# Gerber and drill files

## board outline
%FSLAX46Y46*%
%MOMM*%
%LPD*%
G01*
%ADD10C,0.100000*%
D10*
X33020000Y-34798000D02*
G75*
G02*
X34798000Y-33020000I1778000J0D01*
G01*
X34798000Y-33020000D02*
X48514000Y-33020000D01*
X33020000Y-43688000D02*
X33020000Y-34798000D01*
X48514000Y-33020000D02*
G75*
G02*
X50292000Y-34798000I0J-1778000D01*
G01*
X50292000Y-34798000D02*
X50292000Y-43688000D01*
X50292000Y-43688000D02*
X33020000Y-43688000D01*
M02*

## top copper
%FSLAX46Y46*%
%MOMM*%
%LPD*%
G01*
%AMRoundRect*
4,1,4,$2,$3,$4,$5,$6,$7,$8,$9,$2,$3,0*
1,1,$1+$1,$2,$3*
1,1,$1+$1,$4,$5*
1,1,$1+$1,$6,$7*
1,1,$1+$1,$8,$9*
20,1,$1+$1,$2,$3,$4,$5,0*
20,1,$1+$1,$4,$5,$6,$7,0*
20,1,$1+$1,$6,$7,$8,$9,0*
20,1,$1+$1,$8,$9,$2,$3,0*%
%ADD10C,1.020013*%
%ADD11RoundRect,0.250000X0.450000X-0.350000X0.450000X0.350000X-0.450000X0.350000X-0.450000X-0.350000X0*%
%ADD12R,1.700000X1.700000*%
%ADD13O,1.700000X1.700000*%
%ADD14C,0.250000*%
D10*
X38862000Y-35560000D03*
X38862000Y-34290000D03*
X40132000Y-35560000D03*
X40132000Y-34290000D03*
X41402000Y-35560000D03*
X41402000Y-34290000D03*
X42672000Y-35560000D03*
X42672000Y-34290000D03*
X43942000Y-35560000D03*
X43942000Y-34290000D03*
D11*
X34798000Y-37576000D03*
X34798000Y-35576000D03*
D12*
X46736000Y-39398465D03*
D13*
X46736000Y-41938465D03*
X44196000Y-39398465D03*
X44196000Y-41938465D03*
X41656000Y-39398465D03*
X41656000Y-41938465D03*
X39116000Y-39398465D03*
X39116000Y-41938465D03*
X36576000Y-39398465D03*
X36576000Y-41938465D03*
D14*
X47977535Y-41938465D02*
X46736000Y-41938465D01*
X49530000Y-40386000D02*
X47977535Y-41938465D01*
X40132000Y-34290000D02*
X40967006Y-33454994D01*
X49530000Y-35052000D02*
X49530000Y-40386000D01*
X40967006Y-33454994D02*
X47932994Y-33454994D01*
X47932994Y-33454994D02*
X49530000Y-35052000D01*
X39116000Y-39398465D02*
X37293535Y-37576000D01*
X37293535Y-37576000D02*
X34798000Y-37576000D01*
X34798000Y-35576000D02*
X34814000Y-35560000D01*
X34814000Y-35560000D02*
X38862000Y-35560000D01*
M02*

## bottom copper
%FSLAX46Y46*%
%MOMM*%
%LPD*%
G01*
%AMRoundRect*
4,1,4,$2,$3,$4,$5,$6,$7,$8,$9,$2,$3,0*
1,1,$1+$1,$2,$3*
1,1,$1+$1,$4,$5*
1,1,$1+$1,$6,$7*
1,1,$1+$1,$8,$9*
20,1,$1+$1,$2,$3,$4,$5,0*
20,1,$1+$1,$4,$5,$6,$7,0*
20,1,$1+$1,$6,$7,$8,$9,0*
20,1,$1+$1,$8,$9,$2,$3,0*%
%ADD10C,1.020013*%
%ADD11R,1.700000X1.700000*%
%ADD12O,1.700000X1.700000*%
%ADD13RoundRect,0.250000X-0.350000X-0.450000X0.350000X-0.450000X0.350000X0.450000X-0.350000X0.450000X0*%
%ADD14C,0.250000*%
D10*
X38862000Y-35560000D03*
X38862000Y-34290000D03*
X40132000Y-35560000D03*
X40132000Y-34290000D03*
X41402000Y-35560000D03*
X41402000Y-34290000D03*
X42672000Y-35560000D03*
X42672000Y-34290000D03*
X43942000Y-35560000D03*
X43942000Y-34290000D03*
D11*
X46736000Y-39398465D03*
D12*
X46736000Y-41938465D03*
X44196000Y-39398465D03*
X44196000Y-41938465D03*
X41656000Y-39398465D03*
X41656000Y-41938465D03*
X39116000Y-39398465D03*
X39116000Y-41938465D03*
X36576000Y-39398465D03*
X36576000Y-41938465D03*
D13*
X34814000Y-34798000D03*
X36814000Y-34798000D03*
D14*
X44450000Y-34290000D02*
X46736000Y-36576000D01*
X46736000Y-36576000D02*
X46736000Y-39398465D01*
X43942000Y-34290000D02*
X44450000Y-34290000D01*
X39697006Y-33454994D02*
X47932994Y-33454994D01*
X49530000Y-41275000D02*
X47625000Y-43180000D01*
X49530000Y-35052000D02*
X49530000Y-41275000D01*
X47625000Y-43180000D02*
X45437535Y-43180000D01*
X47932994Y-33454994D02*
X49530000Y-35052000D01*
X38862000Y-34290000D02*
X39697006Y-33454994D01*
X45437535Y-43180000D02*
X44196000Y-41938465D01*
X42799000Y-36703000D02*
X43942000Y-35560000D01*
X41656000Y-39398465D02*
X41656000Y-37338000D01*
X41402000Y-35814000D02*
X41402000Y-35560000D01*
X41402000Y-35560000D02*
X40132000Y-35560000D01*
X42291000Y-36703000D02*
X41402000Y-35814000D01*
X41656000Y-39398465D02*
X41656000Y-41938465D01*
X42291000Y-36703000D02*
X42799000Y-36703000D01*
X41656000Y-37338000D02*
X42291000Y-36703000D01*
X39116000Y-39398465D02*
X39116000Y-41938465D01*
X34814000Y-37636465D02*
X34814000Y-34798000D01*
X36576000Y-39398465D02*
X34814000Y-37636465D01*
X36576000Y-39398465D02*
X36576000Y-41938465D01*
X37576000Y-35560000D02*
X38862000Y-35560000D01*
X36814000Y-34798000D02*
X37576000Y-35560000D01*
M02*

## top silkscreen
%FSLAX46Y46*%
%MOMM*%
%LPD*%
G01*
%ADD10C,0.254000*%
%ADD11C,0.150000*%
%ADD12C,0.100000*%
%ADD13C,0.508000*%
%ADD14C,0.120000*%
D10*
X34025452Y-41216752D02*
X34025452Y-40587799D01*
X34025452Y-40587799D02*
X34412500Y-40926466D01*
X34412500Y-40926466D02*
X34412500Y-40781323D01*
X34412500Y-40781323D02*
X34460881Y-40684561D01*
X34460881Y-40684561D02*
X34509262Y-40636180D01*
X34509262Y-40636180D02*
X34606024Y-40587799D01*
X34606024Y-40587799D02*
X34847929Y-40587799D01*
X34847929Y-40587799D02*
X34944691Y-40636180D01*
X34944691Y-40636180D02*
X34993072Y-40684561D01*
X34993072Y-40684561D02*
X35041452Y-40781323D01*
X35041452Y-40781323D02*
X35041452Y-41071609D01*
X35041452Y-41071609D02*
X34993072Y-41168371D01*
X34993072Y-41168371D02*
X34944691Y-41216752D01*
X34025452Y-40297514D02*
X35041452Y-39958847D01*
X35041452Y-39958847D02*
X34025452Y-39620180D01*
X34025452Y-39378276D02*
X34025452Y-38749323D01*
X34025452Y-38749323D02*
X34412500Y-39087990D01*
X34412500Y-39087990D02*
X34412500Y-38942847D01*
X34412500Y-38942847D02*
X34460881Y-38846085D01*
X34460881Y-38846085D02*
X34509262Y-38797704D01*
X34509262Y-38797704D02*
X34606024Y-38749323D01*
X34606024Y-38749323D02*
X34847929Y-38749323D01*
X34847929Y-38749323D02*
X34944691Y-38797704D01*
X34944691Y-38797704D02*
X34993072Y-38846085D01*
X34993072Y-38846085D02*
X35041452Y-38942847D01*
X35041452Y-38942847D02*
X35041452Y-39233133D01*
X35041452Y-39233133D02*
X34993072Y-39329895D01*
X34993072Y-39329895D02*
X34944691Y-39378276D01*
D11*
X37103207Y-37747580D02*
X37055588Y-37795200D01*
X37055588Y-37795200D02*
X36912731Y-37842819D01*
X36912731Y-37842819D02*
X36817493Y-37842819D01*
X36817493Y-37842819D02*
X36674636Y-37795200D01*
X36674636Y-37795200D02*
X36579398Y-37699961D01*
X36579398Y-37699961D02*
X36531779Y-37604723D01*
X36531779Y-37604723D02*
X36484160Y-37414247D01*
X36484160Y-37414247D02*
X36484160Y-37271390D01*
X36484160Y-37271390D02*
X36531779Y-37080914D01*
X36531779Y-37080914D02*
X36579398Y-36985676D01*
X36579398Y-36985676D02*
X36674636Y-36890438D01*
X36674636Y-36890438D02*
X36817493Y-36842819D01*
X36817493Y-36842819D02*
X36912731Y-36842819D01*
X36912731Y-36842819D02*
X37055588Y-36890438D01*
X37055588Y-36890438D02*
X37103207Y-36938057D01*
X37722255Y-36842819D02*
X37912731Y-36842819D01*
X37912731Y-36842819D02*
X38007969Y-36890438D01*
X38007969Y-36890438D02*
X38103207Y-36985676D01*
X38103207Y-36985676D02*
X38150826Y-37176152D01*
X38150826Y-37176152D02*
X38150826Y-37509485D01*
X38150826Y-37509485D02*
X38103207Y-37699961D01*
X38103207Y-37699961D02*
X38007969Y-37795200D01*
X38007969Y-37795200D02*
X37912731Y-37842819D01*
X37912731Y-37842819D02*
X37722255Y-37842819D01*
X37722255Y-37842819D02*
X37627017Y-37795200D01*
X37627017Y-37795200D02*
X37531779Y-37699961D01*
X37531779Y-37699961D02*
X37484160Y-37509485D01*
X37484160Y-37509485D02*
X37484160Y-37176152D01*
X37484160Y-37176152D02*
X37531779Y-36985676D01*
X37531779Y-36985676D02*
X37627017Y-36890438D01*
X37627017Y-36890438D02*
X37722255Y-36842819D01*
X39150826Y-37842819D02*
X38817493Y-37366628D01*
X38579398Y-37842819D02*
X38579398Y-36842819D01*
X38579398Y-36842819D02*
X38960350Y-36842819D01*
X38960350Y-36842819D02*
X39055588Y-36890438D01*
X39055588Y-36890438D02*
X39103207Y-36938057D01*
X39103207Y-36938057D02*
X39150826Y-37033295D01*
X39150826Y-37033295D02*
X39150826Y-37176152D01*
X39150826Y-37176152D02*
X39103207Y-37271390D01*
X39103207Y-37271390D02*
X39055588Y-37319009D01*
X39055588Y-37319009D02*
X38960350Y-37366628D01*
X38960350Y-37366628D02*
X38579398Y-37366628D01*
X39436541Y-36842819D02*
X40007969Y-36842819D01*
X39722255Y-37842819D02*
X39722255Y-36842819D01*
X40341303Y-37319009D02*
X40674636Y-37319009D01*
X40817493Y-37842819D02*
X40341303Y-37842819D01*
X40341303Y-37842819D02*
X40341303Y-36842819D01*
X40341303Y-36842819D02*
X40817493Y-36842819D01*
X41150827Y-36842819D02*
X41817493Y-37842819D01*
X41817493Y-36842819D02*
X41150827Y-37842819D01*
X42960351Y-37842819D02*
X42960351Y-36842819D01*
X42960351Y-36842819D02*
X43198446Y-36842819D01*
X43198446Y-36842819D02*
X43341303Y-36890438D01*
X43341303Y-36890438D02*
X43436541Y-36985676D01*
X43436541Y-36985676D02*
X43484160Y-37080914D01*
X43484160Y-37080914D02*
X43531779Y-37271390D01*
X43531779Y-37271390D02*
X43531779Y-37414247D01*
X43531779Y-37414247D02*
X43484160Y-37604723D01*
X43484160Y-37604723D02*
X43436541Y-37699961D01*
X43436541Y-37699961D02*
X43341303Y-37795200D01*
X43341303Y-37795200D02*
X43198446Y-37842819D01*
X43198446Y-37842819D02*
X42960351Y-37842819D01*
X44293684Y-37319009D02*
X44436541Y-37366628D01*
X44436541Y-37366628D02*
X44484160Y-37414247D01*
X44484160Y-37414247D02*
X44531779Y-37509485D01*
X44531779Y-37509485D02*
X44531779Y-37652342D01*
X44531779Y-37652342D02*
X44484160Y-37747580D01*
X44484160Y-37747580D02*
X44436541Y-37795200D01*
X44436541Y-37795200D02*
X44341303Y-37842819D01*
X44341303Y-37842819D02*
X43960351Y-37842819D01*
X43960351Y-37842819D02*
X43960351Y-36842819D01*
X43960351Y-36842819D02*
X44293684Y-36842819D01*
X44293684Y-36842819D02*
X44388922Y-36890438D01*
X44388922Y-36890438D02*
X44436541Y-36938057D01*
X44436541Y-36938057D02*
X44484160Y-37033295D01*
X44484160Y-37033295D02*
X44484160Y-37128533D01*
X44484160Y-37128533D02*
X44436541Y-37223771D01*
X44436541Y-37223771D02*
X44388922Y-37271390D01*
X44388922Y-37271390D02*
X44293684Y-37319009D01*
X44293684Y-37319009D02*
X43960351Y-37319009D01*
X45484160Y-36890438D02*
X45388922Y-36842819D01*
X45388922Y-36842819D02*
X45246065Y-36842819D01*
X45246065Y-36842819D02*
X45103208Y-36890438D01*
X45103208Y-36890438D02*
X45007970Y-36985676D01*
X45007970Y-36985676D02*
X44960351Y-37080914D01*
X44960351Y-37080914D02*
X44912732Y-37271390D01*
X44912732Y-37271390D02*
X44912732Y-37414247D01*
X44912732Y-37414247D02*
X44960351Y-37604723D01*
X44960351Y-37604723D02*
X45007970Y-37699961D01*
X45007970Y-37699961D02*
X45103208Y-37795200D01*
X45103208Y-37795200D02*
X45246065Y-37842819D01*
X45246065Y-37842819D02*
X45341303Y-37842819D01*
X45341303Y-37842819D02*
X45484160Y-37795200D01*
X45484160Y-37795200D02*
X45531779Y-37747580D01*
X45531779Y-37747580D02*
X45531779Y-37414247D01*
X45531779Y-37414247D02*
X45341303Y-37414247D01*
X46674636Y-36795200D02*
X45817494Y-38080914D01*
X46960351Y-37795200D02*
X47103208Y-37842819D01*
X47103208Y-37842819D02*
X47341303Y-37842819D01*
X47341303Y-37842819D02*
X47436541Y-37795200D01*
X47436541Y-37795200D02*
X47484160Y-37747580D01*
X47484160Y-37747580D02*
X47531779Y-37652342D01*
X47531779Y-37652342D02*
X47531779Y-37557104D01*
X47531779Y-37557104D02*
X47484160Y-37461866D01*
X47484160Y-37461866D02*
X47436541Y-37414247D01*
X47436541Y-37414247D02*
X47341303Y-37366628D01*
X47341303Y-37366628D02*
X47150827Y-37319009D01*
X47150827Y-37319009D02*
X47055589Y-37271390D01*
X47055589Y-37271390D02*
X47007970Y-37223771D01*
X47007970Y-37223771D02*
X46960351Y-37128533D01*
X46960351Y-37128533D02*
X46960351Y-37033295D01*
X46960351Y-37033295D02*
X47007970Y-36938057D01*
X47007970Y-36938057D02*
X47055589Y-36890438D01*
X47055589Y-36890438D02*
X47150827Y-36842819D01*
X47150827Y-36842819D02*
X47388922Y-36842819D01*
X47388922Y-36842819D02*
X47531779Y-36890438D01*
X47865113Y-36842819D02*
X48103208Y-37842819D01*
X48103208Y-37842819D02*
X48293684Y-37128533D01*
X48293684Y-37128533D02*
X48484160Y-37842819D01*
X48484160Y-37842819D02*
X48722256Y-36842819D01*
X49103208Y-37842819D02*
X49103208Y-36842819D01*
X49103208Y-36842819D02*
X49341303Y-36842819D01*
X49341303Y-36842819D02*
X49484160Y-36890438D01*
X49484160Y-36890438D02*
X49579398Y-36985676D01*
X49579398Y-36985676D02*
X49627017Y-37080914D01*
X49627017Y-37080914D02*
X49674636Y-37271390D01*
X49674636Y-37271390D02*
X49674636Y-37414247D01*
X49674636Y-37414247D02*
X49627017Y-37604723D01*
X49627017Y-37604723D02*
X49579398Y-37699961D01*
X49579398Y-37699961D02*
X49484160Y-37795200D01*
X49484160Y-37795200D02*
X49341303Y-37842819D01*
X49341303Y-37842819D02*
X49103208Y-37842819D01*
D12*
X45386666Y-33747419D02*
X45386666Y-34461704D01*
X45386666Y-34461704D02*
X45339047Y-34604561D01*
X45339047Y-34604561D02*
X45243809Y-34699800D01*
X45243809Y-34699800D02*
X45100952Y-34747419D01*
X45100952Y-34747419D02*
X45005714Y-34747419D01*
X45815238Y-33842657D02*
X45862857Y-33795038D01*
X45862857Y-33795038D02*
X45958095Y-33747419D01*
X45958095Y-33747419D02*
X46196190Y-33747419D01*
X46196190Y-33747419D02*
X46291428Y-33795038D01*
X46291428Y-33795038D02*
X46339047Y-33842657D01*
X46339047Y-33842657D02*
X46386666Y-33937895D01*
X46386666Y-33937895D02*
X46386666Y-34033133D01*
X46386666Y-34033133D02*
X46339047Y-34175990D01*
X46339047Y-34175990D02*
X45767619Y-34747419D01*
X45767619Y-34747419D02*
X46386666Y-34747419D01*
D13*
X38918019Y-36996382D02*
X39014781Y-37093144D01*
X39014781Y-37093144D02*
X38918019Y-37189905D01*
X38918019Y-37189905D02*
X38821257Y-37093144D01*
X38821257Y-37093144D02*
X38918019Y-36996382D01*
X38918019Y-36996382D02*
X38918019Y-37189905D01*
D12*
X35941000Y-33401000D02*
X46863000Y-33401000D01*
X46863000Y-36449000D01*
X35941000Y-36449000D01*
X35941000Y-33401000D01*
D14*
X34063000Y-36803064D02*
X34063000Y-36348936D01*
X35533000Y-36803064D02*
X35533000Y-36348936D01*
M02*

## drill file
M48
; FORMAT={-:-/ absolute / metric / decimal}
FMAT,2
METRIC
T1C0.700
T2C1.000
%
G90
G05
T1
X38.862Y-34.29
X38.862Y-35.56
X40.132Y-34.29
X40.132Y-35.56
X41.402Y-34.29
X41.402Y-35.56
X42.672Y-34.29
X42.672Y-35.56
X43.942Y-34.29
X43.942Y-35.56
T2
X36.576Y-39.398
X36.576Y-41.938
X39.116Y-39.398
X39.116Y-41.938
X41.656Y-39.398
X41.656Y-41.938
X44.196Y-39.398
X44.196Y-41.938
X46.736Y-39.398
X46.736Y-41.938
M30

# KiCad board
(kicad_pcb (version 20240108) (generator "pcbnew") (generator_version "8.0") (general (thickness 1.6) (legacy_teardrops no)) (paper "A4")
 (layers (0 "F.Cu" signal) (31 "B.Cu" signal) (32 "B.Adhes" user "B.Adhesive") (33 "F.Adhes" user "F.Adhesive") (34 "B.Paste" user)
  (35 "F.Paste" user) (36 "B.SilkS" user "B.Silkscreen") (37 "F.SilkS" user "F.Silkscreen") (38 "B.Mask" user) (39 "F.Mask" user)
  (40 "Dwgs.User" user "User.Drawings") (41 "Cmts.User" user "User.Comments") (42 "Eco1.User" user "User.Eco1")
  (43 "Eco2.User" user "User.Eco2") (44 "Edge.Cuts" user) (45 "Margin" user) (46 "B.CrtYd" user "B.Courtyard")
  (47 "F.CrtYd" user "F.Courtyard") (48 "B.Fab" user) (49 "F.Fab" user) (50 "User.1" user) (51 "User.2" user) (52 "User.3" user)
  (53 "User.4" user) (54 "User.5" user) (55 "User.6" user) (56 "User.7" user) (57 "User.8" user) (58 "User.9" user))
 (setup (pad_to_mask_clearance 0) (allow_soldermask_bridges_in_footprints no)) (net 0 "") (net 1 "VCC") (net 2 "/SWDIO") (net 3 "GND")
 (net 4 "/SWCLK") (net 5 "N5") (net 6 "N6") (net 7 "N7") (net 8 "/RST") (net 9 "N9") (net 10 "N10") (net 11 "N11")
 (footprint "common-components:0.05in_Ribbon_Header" (layer "F.Cu") (at 41.402 34.925)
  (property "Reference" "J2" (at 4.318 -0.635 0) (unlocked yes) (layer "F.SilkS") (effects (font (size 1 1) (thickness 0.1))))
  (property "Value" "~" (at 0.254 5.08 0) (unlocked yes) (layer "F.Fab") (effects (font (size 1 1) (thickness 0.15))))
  (fp_rect (start -5.461 -1.524) (end 5.461 1.524) (stroke (width 0.1) (type default)) (fill none) (layer "F.SilkS"))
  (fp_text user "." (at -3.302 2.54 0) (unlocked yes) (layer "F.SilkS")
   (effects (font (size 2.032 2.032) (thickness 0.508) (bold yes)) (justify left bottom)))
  (pad "1" thru_hole circle (at -2.54 0.635) (size 1.020013 1.020013) (drill 0.699999) (layers "*.Cu" "*.Mask") (remove_unused_layers no)
   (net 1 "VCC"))
  (pad "2" thru_hole circle (at -2.54 -0.635) (size 1.020013 1.020013) (drill 0.699999) (layers "*.Cu" "*.Mask") (remove_unused_layers no)
   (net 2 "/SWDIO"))
  (pad "3" thru_hole circle (at -1.27 0.635) (size 1.020013 1.020013) (drill 0.699999) (layers "*.Cu" "*.Mask") (remove_unused_layers no)
   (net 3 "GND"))
  (pad "4" thru_hole circle (at -1.27 -0.635) (size 1.020013 1.020013) (drill 0.699999) (layers "*.Cu" "*.Mask") (remove_unused_layers no)
   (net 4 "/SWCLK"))
  (pad "5" thru_hole circle (at 0 0.635) (size 1.020013 1.020013) (drill 0.699999) (layers "*.Cu" "*.Mask") (remove_unused_layers no)
   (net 3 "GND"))
  (pad "6" thru_hole circle (at 0 -0.635) (size 1.020013 1.020013) (drill 0.699999) (layers "*.Cu" "*.Mask") (remove_unused_layers no)
   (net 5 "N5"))
  (pad "7" thru_hole circle (at 1.27 0.635) (size 1.020013 1.020013) (drill 0.699999) (layers "*.Cu" "*.Mask") (remove_unused_layers no)
   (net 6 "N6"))
  (pad "8" thru_hole circle (at 1.27 -0.635) (size 1.020013 1.020013) (drill 0.699999) (layers "*.Cu" "*.Mask") (remove_unused_layers no)
   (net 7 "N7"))
  (pad "9" thru_hole circle (at 2.54 0.635) (size 1.020013 1.020013) (drill 0.699999) (layers "*.Cu" "*.Mask") (remove_unused_layers no)
   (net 3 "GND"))
  (pad "10" thru_hole circle (at 2.54 -0.635) (size 1.020013 1.020013) (drill 0.699999) (layers "*.Cu" "*.Mask") (remove_unused_layers no)
   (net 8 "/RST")))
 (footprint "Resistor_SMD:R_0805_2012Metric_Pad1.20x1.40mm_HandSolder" (layer "F.Cu") (at 34.798 36.576 90)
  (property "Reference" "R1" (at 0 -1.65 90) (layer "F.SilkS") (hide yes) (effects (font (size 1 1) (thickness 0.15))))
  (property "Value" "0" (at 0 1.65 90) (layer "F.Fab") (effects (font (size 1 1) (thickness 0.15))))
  (fp_line (start -0.227064 -0.735) (end 0.227064 -0.735) (stroke (width 0.12) (type solid)) (layer "F.SilkS"))
  (fp_line (start -0.227064 0.735) (end 0.227064 0.735) (stroke (width 0.12) (type solid)) (layer "F.SilkS"))
  (pad "1" smd roundrect (at -1 0 90) (size 1.2 1.4) (layers "F.Cu" "F.Paste" "F.Mask") (roundrect_rratio 0.208333) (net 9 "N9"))
  (pad "2" smd roundrect (at 1 0 90) (size 1.2 1.4) (layers "F.Cu" "F.Paste" "F.Mask") (roundrect_rratio 0.208333) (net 1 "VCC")))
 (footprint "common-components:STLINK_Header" (layer "B.Cu") (at 41.656 40.668465 180)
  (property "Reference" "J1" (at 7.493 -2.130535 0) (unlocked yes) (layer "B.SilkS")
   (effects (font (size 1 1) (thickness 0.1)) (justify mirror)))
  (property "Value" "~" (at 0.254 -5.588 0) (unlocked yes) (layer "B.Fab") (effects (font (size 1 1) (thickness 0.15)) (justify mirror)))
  (pad "1" thru_hole rect (at -5.08 1.27 90) (size 1.7 1.7) (drill 1) (layers "*.Cu" "*.Mask") (remove_unused_layers no) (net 8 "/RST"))
  (pad "2" thru_hole oval (at -5.08 -1.27 90) (size 1.7 1.7) (drill 1) (layers "*.Cu" "*.Mask") (remove_unused_layers no) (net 4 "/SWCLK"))
  (pad "3" thru_hole oval (at -2.54 1.27 90) (size 1.7 1.7) (drill 1) (layers "*.Cu" "*.Mask") (remove_unused_layers no) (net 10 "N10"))
  (pad "4" thru_hole oval (at -2.54 -1.27 90) (size 1.7 1.7) (drill 1) (layers "*.Cu" "*.Mask") (remove_unused_layers no) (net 2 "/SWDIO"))
  (pad "5" thru_hole oval (at 0 1.27 90) (size 1.7 1.7) (drill 1) (layers "*.Cu" "*.Mask") (remove_unused_layers no) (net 3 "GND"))
  (pad "6" thru_hole oval (at 0 -1.27 90) (size 1.7 1.7) (drill 1) (layers "*.Cu" "*.Mask") (remove_unused_layers no) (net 3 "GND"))
  (pad "7" thru_hole oval (at 2.54 1.27 90) (size 1.7 1.7) (drill 1) (layers "*.Cu" "*.Mask") (remove_unused_layers no) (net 9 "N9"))
  (pad "8" thru_hole oval (at 2.54 -1.27 90) (size 1.7 1.7) (drill 1) (layers "*.Cu" "*.Mask") (remove_unused_layers no) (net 9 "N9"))
  (pad "9" thru_hole oval (at 5.08 1.27 90) (size 1.7 1.7) (drill 1) (layers "*.Cu" "*.Mask") (remove_unused_layers no) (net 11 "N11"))
  (pad "10" thru_hole oval (at 5.08 -1.27 90) (size 1.7 1.7) (drill 1) (layers "*.Cu" "*.Mask") (remove_unused_layers no) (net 11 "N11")))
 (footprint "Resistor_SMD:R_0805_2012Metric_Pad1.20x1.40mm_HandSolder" (layer "B.Cu") (at 35.814 34.798)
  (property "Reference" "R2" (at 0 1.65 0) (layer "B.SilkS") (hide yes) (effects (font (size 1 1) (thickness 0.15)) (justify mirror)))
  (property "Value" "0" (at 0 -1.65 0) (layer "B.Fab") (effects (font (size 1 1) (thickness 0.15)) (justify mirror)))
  (pad "1" smd roundrect (at -1 0) (size 1.2 1.4) (layers "B.Cu" "B.Paste" "B.Mask") (roundrect_rratio 0.208333) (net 11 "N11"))
  (pad "2" smd roundrect (at 1 0) (size 1.2 1.4) (layers "B.Cu" "B.Paste" "B.Mask") (roundrect_rratio 0.208333) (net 1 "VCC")))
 (gr_arc (start 33.02 34.798) (mid 33.540764 33.540764) (end 34.798 33.02) (locked yes) (stroke (width 0.1) (type default))
  (layer "Edge.Cuts"))
 (gr_line (start 34.798 33.02) (end 48.514 33.02) (locked yes) (stroke (width 0.1) (type default)) (layer "Edge.Cuts"))
 (gr_line (start 33.02 43.688) (end 33.02 34.798) (locked yes) (stroke (width 0.1) (type default)) (layer "Edge.Cuts"))
 (gr_arc (start 48.514 33.02) (mid 49.771236 33.540764) (end 50.292 34.798) (locked yes) (stroke (width 0.1) (type default))
  (layer "Edge.Cuts"))
 (gr_line (start 50.292 34.798) (end 50.292 43.688) (locked yes) (stroke (width 0.1) (type default)) (layer "Edge.Cuts"))
 (gr_line (start 50.292 43.688) (end 33.02 43.688) (locked yes) (stroke (width 0.1) (type default)) (layer "Edge.Cuts"))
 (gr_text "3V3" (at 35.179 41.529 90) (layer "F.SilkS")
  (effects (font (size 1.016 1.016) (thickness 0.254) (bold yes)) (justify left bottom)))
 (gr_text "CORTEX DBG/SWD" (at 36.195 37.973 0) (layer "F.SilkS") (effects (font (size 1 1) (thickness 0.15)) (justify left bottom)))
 (segment (start 44.45 34.29) (end 46.736 36.576) (width 0.25) (layer "B.Cu") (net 8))
 (segment (start 46.736 36.576) (end 46.736 39.398465) (width 0.25) (layer "B.Cu") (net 8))
 (segment (start 43.942 34.29) (end 44.45 34.29) (width 0.25) (layer "B.Cu") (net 8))
 (segment (start 47.977535 41.938465) (end 46.736 41.938465) (width 0.25) (layer "F.Cu") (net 4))
 (segment (start 49.53 40.386) (end 47.977535 41.938465) (width 0.25) (layer "F.Cu") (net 4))
 (segment (start 40.132 34.29) (end 40.967006 33.454994) (width 0.25) (layer "F.Cu") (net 4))
 (segment (start 49.53 35.052) (end 49.53 40.386) (width 0.25) (layer "F.Cu") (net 4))
 (segment (start 40.967006 33.454994) (end 47.932994 33.454994) (width 0.25) (layer "F.Cu") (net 4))
 (segment (start 47.932994 33.454994) (end 49.53 35.052) (width 0.25) (layer "F.Cu") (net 4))
 (segment (start 39.697006 33.454994) (end 47.932994 33.454994) (width 0.25) (layer "B.Cu") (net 2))
 (segment (start 49.53 41.275) (end 47.625 43.18) (width 0.25) (layer "B.Cu") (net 2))
 (segment (start 49.53 35.052) (end 49.53 41.275) (width 0.25) (layer "B.Cu") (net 2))
 (segment (start 47.625 43.18) (end 45.437535 43.18) (width 0.25) (layer "B.Cu") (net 2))
 (segment (start 47.932994 33.454994) (end 49.53 35.052) (width 0.25) (layer "B.Cu") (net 2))
 (segment (start 38.862 34.29) (end 39.697006 33.454994) (width 0.25) (layer "B.Cu") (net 2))
 (segment (start 45.437535 43.18) (end 44.196 41.938465) (width 0.25) (layer "B.Cu") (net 2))
 (segment (start 42.799 36.703) (end 43.942 35.56) (width 0.25) (layer "B.Cu") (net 3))
 (segment (start 41.656 39.398465) (end 41.656 37.338) (width 0.25) (layer "B.Cu") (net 3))
 (segment (start 41.402 35.814) (end 41.402 35.56) (width 0.25) (layer "B.Cu") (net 3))
 (segment (start 41.402 35.56) (end 40.132 35.56) (width 0.25) (layer "B.Cu") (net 3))
 (segment (start 42.291 36.703) (end 41.402 35.814) (width 0.25) (layer "B.Cu") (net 3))
 (segment (start 41.656 39.398465) (end 41.656 41.938465) (width 0.25) (layer "B.Cu") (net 3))
 (segment (start 42.291 36.703) (end 42.799 36.703) (width 0.25) (layer "B.Cu") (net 3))
 (segment (start 41.656 37.338) (end 42.291 36.703) (width 0.25) (layer "B.Cu") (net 3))
 (segment (start 39.116 39.398465) (end 37.293535 37.576) (width 0.25) (layer "F.Cu") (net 9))
 (segment (start 37.293535 37.576) (end 34.798 37.576) (width 0.25) (layer "F.Cu") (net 9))
 (segment (start 39.116 39.398465) (end 39.116 41.938465) (width 0.25) (layer "B.Cu") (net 9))
 (segment (start 34.814 37.636465) (end 34.814 34.798) (width 0.25) (layer "B.Cu") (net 11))
 (segment (start 36.576 39.398465) (end 34.814 37.636465) (width 0.25) (layer "B.Cu") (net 11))
 (segment (start 36.576 39.398465) (end 36.576 41.938465) (width 0.25) (layer "B.Cu") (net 11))
 (segment (start 34.798 35.576) (end 34.814 35.56) (width 0.25) (layer "F.Cu") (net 1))
 (segment (start 34.814 35.56) (end 38.862 35.56) (width 0.25) (layer "F.Cu") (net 1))
 (segment (start 37.576 35.56) (end 38.862 35.56) (width 0.25) (layer "B.Cu") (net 1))
 (segment (start 36.814 34.798) (end 37.576 35.56) (width 0.25) (layer "B.Cu") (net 1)))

